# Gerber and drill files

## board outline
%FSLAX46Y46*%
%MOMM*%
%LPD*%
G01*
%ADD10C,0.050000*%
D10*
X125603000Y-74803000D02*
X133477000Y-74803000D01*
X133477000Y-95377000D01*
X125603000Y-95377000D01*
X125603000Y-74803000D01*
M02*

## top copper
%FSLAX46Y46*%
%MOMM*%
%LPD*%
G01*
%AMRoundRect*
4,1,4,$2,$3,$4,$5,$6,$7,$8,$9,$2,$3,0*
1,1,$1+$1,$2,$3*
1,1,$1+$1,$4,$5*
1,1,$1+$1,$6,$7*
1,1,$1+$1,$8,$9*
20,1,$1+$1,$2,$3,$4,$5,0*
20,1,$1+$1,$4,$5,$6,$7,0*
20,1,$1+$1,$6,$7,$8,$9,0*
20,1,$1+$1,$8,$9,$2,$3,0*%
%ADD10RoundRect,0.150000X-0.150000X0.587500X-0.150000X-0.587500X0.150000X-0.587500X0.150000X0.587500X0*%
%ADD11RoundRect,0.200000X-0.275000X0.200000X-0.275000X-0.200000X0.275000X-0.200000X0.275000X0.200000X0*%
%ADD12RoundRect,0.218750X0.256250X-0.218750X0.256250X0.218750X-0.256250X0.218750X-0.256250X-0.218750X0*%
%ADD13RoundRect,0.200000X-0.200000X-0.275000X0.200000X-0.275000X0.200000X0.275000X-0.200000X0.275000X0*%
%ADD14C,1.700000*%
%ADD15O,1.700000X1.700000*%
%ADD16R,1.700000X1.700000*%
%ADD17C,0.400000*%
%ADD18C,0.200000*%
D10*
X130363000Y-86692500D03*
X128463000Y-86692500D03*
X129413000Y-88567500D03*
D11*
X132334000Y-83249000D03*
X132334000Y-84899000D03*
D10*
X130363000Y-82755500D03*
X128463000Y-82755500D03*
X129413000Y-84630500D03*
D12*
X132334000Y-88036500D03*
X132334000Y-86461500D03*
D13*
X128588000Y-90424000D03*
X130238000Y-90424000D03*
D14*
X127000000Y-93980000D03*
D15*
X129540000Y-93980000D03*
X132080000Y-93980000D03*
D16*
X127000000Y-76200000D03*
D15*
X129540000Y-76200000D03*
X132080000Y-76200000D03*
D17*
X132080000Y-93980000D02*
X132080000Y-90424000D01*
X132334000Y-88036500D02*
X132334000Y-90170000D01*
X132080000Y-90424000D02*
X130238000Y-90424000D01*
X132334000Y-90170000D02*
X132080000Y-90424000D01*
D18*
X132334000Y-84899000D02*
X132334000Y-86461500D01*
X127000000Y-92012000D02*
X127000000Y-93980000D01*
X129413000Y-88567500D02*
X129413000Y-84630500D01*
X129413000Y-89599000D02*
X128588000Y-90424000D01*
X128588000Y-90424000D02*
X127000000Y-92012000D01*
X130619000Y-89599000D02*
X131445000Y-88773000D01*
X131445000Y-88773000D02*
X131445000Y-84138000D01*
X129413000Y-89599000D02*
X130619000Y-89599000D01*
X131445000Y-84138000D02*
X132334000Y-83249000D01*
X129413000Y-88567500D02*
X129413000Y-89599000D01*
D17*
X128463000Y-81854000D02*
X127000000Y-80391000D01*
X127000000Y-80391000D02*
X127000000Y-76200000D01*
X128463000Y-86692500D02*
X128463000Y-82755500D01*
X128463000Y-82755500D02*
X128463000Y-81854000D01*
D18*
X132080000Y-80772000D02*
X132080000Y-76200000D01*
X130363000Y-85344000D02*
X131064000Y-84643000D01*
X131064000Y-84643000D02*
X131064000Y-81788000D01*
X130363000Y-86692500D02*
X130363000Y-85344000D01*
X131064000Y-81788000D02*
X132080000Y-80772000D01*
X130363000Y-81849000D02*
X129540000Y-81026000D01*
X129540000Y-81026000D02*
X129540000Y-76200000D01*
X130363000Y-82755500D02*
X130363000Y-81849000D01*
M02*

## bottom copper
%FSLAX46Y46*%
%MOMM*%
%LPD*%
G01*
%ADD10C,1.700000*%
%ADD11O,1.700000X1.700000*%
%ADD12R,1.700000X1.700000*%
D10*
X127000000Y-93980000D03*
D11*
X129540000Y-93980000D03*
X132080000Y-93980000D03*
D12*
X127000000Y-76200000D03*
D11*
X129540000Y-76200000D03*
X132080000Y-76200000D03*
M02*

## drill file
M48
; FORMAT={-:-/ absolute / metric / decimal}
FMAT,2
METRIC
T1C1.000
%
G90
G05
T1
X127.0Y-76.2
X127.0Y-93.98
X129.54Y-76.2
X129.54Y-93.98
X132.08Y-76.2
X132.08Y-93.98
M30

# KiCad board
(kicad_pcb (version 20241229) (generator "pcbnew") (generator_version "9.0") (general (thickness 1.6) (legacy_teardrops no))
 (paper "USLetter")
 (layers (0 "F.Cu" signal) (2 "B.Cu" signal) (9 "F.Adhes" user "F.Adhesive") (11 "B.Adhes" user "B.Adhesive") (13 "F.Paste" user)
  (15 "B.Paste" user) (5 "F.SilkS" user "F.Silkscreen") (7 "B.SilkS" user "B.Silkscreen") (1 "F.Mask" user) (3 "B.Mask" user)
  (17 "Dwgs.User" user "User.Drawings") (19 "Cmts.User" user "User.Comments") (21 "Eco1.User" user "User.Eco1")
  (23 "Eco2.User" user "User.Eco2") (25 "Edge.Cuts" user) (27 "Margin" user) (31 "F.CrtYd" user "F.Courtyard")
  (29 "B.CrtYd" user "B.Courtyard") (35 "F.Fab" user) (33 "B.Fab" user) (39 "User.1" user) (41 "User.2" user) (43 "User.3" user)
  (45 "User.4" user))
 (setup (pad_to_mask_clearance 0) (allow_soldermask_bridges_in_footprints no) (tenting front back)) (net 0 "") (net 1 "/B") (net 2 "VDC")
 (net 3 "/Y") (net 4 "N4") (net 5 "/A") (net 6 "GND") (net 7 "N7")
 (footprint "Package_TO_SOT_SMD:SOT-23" (layer "F.Cu") (at 129.413 87.63 -90)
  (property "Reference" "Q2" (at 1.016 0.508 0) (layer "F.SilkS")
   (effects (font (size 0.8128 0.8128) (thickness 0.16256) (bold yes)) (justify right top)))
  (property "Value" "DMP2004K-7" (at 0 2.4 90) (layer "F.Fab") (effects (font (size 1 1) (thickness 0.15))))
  (pad "1" smd roundrect (at -0.9375 -0.95 270) (size 1.475 0.6) (layers "F.Cu" "F.Mask" "F.Paste") (roundrect_rratio 0.25) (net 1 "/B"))
  (pad "2" smd roundrect (at -0.9375 0.95 270) (size 1.475 0.6) (layers "F.Cu" "F.Mask" "F.Paste") (roundrect_rratio 0.25) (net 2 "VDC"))
  (pad "3" smd roundrect (at 0.9375 0 270) (size 1.475 0.6) (layers "F.Cu" "F.Mask" "F.Paste") (roundrect_rratio 0.25) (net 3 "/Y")))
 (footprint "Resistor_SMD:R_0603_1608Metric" (layer "F.Cu") (at 132.334 84.074 -90)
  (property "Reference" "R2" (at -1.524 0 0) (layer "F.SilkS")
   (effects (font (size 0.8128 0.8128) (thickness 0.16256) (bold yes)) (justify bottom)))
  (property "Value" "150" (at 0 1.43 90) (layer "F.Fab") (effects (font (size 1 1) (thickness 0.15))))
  (pad "1" smd roundrect (at -0.825 0 270) (size 0.8 0.95) (layers "F.Cu" "F.Mask" "F.Paste") (roundrect_rratio 0.25) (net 3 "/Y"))
  (pad "2" smd roundrect (at 0.825 0 270) (size 0.8 0.95) (layers "F.Cu" "F.Mask" "F.Paste") (roundrect_rratio 0.25) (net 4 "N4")))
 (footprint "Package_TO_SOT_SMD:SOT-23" (layer "F.Cu") (at 129.413 83.693 -90)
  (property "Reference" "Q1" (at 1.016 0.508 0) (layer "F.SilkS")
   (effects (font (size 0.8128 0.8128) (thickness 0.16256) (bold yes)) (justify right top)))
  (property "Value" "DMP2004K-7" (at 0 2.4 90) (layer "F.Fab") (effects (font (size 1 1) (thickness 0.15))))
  (pad "1" smd roundrect (at -0.9375 -0.95 270) (size 1.475 0.6) (layers "F.Cu" "F.Mask" "F.Paste") (roundrect_rratio 0.25) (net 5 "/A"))
  (pad "2" smd roundrect (at -0.9375 0.95 270) (size 1.475 0.6) (layers "F.Cu" "F.Mask" "F.Paste") (roundrect_rratio 0.25) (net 2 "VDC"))
  (pad "3" smd roundrect (at 0.9375 0 270) (size 1.475 0.6) (layers "F.Cu" "F.Mask" "F.Paste") (roundrect_rratio 0.25) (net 3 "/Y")))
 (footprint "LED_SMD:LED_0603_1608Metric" (layer "F.Cu") (at 132.334 87.249 90)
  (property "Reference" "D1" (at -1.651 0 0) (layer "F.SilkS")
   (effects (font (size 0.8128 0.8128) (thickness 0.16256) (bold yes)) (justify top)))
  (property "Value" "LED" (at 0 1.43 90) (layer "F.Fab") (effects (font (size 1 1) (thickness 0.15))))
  (pad "1" smd roundrect (at -0.7875 0 90) (size 0.875 0.95) (layers "F.Cu" "F.Mask" "F.Paste") (roundrect_rratio 0.25) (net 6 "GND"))
  (pad "2" smd roundrect (at 0.7875 0 90) (size 0.875 0.95) (layers "F.Cu" "F.Mask" "F.Paste") (roundrect_rratio 0.25) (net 4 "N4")))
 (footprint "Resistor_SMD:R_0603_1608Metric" (layer "F.Cu") (at 129.413 90.424)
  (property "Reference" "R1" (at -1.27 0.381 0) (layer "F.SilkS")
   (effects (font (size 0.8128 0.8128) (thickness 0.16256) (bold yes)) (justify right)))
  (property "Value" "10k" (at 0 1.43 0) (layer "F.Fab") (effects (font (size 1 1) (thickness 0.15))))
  (pad "1" smd roundrect (at -0.825 0) (size 0.8 0.95) (layers "F.Cu" "F.Mask" "F.Paste") (roundrect_rratio 0.25) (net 3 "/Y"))
  (pad "2" smd roundrect (at 0.825 0) (size 0.8 0.95) (layers "F.Cu" "F.Mask" "F.Paste") (roundrect_rratio 0.25) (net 6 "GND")))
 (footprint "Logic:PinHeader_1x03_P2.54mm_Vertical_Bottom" (layer "B.Cu") (at 127 93.98 -90)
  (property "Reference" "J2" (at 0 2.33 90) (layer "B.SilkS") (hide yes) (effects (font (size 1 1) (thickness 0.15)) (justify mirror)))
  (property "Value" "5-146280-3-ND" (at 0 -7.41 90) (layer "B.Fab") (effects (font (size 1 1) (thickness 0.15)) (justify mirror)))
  (pad "1" thru_hole circle (at 0 0 270) (size 1.7 1.7) (drill 1) (layers "*.Cu" "*.Mask") (remove_unused_layers no) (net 3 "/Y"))
  (pad "2" thru_hole oval (at 0 -2.54 270) (size 1.7 1.7) (drill 1) (layers "*.Cu" "*.Mask") (remove_unused_layers no) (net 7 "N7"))
  (pad "3" thru_hole oval (at 0 -5.08 270) (size 1.7 1.7) (drill 1) (layers "*.Cu" "*.Mask") (remove_unused_layers no) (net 6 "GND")))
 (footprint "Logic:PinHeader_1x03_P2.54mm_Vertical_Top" (layer "B.Cu") (at 127 76.2 -90)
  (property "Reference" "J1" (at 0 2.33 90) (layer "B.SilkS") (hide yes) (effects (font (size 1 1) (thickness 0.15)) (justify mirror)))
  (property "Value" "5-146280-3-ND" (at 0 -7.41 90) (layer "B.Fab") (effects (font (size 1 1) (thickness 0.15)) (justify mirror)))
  (pad "1" thru_hole rect (at 0 0 270) (size 1.7 1.7) (drill 1) (layers "*.Cu" "*.Mask") (remove_unused_layers no) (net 2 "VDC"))
  (pad "2" thru_hole oval (at 0 -2.54 270) (size 1.7 1.7) (drill 1) (layers "*.Cu" "*.Mask") (remove_unused_layers no) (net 5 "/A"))
  (pad "3" thru_hole oval (at 0 -5.08 270) (size 1.7 1.7) (drill 1) (layers "*.Cu" "*.Mask") (remove_unused_layers no) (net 1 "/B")))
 (gr_rect (start 125.603 74.803) (end 133.477 95.377) (stroke (width 0.05) (type default)) (fill no) (layer "Edge.Cuts"))
 (segment (start 132.08 93.98) (end 132.08 90.424) (width 0.4) (layer "F.Cu") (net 6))
 (segment (start 132.334 88.0365) (end 132.334 90.17) (width 0.4) (layer "F.Cu") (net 6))
 (segment (start 132.08 90.424) (end 130.238 90.424) (width 0.4) (layer "F.Cu") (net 6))
 (segment (start 132.334 90.17) (end 132.08 90.424) (width 0.4) (layer "F.Cu") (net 6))
 (segment (start 132.334 84.899) (end 132.334 86.4615) (width 0.2) (layer "F.Cu") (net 4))
 (segment (start 127 92.012) (end 127 93.98) (width 0.2) (layer "F.Cu") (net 3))
 (segment (start 129.413 88.5675) (end 129.413 84.6305) (width 0.2) (layer "F.Cu") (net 3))
 (segment (start 129.413 89.599) (end 128.588 90.424) (width 0.2) (layer "F.Cu") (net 3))
 (segment (start 128.588 90.424) (end 127 92.012) (width 0.2) (layer "F.Cu") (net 3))
 (segment (start 130.619 89.599) (end 131.445 88.773) (width 0.2) (layer "F.Cu") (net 3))
 (segment (start 131.445 88.773) (end 131.445 84.138) (width 0.2) (layer "F.Cu") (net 3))
 (segment (start 129.413 89.599) (end 130.619 89.599) (width 0.2) (layer "F.Cu") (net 3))
 (segment (start 131.445 84.138) (end 132.334 83.249) (width 0.2) (layer "F.Cu") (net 3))
 (segment (start 129.413 88.5675) (end 129.413 89.599) (width 0.2) (layer "F.Cu") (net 3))
 (segment (start 128.463 81.854) (end 127 80.391) (width 0.4) (layer "F.Cu") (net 2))
 (segment (start 127 80.391) (end 127 76.2) (width 0.4) (layer "F.Cu") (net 2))
 (segment (start 128.463 86.6925) (end 128.463 82.7555) (width 0.4) (layer "F.Cu") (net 2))
 (segment (start 128.463 82.7555) (end 128.463 81.854) (width 0.4) (layer "F.Cu") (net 2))
 (segment (start 132.08 80.772) (end 132.08 76.2) (width 0.2) (layer "F.Cu") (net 1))
 (segment (start 130.363 85.344) (end 131.064 84.643) (width 0.2) (layer "F.Cu") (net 1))
 (segment (start 131.064 84.643) (end 131.064 81.788) (width 0.2) (layer "F.Cu") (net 1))
 (segment (start 130.363 86.6925) (end 130.363 85.344) (width 0.2) (layer "F.Cu") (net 1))
 (segment (start 131.064 81.788) (end 132.08 80.772) (width 0.2) (layer "F.Cu") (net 1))
 (segment (start 130.363 81.849) (end 129.54 81.026) (width 0.2) (layer "F.Cu") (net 5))
 (segment (start 129.54 81.026) (end 129.54 76.2) (width 0.2) (layer "F.Cu") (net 5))
 (segment (start 130.363 82.7555) (end 130.363 81.849) (width 0.2) (layer "F.Cu") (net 5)))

